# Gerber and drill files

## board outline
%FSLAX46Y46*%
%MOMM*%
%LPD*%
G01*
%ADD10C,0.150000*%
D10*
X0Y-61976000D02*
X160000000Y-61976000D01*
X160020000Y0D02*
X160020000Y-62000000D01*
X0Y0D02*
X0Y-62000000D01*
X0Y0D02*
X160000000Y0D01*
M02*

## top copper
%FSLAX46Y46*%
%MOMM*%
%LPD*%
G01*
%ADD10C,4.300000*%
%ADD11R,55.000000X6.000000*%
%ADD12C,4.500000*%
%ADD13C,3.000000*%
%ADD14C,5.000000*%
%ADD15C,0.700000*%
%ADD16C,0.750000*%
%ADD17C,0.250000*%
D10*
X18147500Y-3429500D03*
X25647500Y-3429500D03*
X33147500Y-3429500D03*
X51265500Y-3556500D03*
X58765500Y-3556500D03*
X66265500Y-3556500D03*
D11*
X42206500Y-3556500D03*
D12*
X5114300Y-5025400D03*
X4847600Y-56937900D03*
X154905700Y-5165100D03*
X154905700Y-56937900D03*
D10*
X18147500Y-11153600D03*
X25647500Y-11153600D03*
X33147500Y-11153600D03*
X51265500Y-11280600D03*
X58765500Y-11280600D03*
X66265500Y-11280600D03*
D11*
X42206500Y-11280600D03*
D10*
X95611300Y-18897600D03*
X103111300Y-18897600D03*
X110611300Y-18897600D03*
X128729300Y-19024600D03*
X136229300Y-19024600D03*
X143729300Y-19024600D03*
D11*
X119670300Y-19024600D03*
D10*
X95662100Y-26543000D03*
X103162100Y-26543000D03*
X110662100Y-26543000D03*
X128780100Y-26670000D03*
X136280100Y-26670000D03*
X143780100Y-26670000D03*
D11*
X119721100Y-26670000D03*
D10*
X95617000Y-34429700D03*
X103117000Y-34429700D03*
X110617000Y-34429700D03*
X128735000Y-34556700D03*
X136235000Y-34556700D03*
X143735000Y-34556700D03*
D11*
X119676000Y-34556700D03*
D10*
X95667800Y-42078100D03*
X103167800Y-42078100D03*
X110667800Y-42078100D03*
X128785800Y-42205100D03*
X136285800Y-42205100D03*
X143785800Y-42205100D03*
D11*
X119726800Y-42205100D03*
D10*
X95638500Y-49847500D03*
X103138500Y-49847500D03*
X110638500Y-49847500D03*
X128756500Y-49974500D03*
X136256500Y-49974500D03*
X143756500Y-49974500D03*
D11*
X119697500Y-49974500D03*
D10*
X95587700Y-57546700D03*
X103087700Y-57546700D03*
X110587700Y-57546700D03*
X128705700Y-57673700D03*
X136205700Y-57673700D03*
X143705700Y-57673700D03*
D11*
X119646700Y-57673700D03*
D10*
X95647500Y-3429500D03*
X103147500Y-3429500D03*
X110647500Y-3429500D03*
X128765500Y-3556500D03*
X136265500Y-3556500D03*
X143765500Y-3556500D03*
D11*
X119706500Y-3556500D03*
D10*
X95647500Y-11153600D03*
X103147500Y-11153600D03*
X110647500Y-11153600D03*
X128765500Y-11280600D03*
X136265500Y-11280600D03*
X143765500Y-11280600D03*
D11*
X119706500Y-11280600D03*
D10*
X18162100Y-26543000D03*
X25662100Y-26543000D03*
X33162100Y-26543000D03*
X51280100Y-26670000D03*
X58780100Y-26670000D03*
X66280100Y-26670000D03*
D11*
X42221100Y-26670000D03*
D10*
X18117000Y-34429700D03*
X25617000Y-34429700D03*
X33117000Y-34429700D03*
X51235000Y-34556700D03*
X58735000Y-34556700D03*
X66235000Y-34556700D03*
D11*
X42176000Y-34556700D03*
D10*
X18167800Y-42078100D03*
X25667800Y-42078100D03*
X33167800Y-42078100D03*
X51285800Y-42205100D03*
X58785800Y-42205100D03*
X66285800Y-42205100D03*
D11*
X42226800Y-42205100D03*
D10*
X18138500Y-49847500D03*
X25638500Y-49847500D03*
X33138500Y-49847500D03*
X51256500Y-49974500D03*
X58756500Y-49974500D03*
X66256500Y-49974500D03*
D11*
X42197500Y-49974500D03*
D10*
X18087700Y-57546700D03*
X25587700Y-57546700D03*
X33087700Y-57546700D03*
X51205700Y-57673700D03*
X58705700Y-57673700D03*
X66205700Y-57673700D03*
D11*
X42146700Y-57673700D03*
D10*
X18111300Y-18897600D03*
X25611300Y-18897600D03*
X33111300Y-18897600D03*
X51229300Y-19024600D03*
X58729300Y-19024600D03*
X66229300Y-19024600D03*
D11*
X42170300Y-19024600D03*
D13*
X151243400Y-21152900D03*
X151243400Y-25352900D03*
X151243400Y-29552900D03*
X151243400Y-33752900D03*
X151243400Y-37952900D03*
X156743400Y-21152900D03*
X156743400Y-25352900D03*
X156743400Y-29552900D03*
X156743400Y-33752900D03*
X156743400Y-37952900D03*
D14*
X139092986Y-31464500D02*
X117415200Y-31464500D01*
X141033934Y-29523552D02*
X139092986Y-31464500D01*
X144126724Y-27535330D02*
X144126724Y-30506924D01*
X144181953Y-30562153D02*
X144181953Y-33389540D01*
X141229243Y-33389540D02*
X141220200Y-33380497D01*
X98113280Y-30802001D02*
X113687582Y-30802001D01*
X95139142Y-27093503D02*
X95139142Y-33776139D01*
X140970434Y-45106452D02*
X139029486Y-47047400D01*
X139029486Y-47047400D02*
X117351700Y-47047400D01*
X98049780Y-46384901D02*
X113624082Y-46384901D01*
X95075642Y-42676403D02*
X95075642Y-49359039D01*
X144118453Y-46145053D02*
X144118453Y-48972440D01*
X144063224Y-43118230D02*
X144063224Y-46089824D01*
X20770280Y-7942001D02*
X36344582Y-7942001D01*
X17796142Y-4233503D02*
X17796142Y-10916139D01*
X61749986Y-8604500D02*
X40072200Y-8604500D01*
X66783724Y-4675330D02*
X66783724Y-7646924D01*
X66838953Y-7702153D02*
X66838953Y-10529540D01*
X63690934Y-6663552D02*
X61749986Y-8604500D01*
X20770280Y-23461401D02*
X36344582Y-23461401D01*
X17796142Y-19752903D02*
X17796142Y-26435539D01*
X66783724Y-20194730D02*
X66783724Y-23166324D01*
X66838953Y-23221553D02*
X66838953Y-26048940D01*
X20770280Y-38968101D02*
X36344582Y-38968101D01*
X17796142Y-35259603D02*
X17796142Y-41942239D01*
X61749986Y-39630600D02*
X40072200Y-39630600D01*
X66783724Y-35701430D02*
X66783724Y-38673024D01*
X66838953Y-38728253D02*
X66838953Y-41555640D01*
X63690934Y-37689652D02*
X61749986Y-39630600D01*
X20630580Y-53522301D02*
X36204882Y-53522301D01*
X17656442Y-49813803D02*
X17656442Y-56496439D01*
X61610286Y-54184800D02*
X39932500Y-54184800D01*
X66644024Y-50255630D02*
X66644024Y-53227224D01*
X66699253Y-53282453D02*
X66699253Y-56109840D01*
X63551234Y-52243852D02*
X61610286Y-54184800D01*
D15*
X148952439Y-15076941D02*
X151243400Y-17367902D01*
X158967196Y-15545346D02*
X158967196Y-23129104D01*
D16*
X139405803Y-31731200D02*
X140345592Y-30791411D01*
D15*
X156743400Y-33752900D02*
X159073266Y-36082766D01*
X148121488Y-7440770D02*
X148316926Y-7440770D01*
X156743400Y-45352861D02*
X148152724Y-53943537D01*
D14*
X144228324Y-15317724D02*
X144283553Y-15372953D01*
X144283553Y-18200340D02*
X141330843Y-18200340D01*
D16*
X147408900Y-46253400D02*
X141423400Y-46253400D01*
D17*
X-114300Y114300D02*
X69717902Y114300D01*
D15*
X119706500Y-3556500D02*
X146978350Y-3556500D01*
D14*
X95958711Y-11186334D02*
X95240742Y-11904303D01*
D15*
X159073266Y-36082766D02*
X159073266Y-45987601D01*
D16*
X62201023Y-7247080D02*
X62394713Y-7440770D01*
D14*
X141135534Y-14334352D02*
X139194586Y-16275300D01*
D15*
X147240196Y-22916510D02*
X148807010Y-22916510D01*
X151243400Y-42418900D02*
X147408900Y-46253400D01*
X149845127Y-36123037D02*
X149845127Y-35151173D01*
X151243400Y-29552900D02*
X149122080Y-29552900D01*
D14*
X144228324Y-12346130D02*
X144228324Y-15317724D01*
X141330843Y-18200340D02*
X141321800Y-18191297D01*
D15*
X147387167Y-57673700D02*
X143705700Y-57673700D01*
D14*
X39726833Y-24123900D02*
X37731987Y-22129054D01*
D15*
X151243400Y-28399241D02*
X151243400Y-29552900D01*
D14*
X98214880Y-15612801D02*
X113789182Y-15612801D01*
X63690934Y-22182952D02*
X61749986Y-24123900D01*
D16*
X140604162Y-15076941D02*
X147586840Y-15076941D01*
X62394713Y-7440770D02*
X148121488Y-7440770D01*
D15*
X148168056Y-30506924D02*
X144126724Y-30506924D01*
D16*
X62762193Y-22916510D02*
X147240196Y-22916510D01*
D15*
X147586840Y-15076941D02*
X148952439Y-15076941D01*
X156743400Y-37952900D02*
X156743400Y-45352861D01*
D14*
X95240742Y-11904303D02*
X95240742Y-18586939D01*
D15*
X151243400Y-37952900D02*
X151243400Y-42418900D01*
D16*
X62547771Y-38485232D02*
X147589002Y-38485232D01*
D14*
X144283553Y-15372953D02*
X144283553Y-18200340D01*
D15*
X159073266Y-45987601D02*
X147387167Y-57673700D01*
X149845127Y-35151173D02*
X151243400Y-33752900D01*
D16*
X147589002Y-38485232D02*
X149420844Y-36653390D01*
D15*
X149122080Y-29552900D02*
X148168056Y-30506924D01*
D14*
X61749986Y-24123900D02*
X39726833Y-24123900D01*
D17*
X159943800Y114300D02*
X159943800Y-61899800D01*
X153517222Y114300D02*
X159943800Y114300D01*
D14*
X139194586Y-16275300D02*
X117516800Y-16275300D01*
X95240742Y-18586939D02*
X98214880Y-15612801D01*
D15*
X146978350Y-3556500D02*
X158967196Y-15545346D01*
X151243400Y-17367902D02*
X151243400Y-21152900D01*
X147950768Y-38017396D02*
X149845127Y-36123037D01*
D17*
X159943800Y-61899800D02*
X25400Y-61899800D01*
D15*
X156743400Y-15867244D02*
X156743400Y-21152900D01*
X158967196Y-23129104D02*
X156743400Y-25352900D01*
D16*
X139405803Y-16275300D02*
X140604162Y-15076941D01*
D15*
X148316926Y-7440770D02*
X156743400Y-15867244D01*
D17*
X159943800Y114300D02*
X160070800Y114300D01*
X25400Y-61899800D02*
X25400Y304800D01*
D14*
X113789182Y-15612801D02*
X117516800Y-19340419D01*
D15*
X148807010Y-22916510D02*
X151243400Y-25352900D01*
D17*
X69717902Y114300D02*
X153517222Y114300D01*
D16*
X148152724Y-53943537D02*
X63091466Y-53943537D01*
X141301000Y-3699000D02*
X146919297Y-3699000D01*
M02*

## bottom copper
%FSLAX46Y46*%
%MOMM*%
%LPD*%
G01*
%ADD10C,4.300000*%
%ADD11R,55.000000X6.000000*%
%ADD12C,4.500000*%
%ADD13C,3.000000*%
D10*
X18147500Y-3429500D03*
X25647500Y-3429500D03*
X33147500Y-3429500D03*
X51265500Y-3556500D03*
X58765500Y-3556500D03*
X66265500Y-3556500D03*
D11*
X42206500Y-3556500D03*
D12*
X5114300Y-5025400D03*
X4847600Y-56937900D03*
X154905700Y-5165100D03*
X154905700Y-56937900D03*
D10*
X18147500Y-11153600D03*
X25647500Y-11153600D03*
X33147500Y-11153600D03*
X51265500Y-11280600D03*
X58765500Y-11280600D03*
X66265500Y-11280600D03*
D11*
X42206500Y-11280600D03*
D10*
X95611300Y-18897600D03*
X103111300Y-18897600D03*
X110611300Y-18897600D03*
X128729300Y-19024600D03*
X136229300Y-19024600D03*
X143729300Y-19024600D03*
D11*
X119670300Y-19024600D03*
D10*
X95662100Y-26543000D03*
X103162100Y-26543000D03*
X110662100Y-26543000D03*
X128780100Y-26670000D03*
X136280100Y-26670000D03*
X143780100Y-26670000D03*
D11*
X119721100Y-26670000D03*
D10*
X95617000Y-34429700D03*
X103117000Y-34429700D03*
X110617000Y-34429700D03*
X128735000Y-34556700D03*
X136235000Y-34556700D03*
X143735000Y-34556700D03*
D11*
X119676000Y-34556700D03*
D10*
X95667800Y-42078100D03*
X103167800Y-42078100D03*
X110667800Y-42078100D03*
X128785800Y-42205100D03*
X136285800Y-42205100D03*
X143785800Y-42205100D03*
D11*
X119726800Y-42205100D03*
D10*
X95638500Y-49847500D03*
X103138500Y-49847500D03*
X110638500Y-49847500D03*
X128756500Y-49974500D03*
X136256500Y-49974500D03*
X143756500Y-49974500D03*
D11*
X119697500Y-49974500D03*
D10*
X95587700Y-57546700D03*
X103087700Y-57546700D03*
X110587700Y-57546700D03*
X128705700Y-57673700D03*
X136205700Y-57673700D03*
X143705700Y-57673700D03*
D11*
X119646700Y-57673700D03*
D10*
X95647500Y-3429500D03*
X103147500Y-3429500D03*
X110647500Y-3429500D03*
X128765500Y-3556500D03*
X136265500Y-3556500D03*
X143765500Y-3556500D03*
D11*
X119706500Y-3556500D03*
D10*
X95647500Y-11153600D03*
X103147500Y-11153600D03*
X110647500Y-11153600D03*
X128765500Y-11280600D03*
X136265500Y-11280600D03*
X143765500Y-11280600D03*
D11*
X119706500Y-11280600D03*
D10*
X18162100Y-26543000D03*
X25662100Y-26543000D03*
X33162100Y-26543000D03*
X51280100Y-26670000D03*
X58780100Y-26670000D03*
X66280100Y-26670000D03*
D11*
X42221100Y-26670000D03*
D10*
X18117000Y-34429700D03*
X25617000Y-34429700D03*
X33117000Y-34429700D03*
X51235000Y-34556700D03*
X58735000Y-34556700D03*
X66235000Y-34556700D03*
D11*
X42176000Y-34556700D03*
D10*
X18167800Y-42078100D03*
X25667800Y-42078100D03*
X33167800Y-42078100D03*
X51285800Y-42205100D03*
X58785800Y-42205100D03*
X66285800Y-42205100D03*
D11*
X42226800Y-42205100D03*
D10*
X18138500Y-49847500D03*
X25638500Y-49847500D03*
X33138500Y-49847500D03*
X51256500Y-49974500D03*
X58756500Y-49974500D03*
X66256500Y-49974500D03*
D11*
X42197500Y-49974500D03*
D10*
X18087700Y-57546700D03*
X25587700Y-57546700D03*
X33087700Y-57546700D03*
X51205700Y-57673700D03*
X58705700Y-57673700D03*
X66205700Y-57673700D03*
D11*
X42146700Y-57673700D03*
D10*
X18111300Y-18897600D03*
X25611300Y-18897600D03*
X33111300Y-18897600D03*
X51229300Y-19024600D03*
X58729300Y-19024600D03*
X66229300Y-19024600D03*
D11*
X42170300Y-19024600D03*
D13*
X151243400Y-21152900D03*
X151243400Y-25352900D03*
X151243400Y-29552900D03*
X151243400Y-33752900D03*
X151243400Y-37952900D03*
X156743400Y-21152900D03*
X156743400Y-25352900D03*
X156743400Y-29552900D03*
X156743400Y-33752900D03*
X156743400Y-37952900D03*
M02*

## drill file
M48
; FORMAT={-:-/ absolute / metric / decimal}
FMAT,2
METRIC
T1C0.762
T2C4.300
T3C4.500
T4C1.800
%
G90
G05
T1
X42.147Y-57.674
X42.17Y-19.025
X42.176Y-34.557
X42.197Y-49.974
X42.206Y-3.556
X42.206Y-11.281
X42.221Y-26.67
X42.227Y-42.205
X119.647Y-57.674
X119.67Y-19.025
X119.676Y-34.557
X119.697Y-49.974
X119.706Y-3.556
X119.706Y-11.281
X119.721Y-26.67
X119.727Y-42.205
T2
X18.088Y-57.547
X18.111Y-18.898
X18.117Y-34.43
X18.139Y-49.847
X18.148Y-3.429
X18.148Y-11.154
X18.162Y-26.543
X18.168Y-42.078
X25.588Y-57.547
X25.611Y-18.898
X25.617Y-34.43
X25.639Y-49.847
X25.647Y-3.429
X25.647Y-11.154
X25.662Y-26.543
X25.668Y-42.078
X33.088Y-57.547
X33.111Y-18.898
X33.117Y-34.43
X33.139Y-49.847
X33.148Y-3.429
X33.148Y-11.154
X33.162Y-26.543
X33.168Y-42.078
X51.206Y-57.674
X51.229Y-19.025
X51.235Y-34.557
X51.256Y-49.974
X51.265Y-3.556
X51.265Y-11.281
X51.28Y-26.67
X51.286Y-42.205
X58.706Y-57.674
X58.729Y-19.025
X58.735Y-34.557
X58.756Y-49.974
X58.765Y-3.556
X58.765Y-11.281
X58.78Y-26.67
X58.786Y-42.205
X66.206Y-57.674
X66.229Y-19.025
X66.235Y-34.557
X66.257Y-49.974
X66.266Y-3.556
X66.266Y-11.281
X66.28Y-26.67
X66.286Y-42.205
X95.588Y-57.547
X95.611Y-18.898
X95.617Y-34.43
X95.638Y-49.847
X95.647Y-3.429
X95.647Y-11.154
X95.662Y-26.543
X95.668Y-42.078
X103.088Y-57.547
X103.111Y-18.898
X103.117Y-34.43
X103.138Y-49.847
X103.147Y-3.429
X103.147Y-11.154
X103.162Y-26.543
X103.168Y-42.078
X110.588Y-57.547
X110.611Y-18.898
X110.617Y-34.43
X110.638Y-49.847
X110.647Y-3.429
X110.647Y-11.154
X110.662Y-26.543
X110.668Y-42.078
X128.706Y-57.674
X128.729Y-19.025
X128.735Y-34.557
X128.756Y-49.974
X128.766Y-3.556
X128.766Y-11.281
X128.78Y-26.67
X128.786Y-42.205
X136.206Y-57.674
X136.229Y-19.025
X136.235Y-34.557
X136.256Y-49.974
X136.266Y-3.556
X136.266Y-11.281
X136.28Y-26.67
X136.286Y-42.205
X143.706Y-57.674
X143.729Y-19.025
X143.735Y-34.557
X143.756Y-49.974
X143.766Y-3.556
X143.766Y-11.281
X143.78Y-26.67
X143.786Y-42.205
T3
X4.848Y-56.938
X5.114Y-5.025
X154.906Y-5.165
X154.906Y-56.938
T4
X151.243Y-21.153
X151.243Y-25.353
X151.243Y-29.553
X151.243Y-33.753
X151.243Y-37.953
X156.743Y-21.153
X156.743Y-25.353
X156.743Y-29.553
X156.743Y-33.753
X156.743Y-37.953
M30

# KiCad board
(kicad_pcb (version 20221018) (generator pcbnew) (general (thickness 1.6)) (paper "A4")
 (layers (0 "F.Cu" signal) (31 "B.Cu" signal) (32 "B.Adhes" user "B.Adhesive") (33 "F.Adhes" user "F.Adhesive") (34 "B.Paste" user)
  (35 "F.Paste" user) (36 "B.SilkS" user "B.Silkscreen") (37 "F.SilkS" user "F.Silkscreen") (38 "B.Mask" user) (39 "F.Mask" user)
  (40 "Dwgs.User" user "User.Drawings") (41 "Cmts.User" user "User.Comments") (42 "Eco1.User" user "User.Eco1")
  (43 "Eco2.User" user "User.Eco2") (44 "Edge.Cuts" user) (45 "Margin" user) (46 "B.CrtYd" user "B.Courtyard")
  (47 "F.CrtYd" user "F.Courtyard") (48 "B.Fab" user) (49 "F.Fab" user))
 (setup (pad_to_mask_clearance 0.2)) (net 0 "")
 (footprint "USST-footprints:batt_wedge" (layer "F.Cu") (at 42.2065 3.5565)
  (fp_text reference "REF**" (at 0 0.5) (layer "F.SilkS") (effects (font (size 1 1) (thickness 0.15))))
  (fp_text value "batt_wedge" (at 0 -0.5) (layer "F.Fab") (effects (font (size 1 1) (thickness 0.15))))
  (pad "" thru_hole circle (at -24.059 -0.127) (size 4.3 4.3) (drill 4.3) (layers "*.Cu" "*.Mask"))
  (pad "" thru_hole circle (at -16.559 -0.127) (size 4.3 4.3) (drill 4.3) (layers "*.Cu" "*.Mask"))
  (pad "" thru_hole circle (at -9.059 -0.127) (size 4.3 4.3) (drill 4.3) (layers "*.Cu" "*.Mask"))
  (pad "" thru_hole circle (at 9.059 0) (size 4.3 4.3) (drill 4.3) (layers "*.Cu" "*.Mask"))
  (pad "" thru_hole circle (at 16.559 0) (size 4.3 4.3) (drill 4.3) (layers "*.Cu" "*.Mask"))
  (pad "" thru_hole circle (at 24.059 0) (size 4.3 4.3) (drill 4.3) (layers "*.Cu" "*.Mask"))
  (pad "1" thru_hole rect (at 0 0) (size 55 6) (drill 0.762) (layers "F.Cu" "F.Paste")))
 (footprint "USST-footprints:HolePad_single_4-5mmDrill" (layer "F.Cu") (at 5.1143 5.0254)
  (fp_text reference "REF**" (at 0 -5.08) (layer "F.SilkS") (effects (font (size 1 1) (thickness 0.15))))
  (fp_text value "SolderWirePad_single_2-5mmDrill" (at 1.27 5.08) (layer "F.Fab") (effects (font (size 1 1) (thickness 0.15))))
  (pad "" thru_hole circle (at 0 0) (size 4.5 4.5) (drill 4.5) (layers "*.Cu" "*.Mask")))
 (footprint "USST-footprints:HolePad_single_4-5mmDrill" (layer "F.Cu") (at 4.8476 56.9379)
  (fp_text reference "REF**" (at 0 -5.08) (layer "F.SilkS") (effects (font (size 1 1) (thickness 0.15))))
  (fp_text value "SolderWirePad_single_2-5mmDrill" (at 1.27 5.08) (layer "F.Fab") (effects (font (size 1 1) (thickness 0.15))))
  (pad "" thru_hole circle (at 0 0) (size 4.5 4.5) (drill 4.5) (layers "*.Cu" "*.Mask")))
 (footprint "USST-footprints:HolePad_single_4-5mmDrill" (layer "F.Cu") (at 154.9057 5.1651)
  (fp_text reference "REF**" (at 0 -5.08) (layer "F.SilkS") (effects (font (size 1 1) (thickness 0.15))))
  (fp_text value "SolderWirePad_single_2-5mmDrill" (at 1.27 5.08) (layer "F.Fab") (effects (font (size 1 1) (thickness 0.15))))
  (pad "" thru_hole circle (at 0 0) (size 4.5 4.5) (drill 4.5) (layers "*.Cu" "*.Mask")))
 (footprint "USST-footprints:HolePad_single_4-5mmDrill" (layer "F.Cu") (at 154.9057 56.9379)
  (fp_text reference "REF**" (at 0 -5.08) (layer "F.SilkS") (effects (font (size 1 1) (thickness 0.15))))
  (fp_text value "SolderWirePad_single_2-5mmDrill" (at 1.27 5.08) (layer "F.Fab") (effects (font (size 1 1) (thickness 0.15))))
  (pad "" thru_hole circle (at 0 0) (size 4.5 4.5) (drill 4.5) (layers "*.Cu" "*.Mask")))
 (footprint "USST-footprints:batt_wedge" (layer "F.Cu") (at 42.2065 11.2806)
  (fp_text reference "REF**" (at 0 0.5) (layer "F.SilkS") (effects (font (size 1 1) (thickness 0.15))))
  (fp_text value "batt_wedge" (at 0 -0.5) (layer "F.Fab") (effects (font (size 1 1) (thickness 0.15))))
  (pad "" thru_hole circle (at -24.059 -0.127) (size 4.3 4.3) (drill 4.3) (layers "*.Cu" "*.Mask"))
  (pad "" thru_hole circle (at -16.559 -0.127) (size 4.3 4.3) (drill 4.3) (layers "*.Cu" "*.Mask"))
  (pad "" thru_hole circle (at -9.059 -0.127) (size 4.3 4.3) (drill 4.3) (layers "*.Cu" "*.Mask"))
  (pad "" thru_hole circle (at 9.059 0) (size 4.3 4.3) (drill 4.3) (layers "*.Cu" "*.Mask"))
  (pad "" thru_hole circle (at 16.559 0) (size 4.3 4.3) (drill 4.3) (layers "*.Cu" "*.Mask"))
  (pad "" thru_hole circle (at 24.059 0) (size 4.3 4.3) (drill 4.3) (layers "*.Cu" "*.Mask"))
  (pad "1" thru_hole rect (at 0 0) (size 55 6) (drill 0.762) (layers "F.Cu" "F.Paste")))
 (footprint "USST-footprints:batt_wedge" (layer "F.Cu") (at 119.6703 19.0246)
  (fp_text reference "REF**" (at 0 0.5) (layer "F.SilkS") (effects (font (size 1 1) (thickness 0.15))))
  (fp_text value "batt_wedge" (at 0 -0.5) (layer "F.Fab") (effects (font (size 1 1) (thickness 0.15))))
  (pad "" thru_hole circle (at -24.059 -0.127) (size 4.3 4.3) (drill 4.3) (layers "*.Cu" "*.Mask"))
  (pad "" thru_hole circle (at -16.559 -0.127) (size 4.3 4.3) (drill 4.3) (layers "*.Cu" "*.Mask"))
  (pad "" thru_hole circle (at -9.059 -0.127) (size 4.3 4.3) (drill 4.3) (layers "*.Cu" "*.Mask"))
  (pad "" thru_hole circle (at 9.059 0) (size 4.3 4.3) (drill 4.3) (layers "*.Cu" "*.Mask"))
  (pad "" thru_hole circle (at 16.559 0) (size 4.3 4.3) (drill 4.3) (layers "*.Cu" "*.Mask"))
  (pad "" thru_hole circle (at 24.059 0) (size 4.3 4.3) (drill 4.3) (layers "*.Cu" "*.Mask"))
  (pad "1" thru_hole rect (at 0 0) (size 55 6) (drill 0.762) (layers "F.Cu" "F.Paste")))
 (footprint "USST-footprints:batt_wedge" (layer "F.Cu") (at 119.7211 26.67)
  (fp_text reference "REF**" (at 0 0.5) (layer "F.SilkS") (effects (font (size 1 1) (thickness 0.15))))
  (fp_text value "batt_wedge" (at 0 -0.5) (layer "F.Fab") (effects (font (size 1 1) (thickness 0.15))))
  (pad "" thru_hole circle (at -24.059 -0.127) (size 4.3 4.3) (drill 4.3) (layers "*.Cu" "*.Mask"))
  (pad "" thru_hole circle (at -16.559 -0.127) (size 4.3 4.3) (drill 4.3) (layers "*.Cu" "*.Mask"))
  (pad "" thru_hole circle (at -9.059 -0.127) (size 4.3 4.3) (drill 4.3) (layers "*.Cu" "*.Mask"))
  (pad "" thru_hole circle (at 9.059 0) (size 4.3 4.3) (drill 4.3) (layers "*.Cu" "*.Mask"))
  (pad "" thru_hole circle (at 16.559 0) (size 4.3 4.3) (drill 4.3) (layers "*.Cu" "*.Mask"))
  (pad "" thru_hole circle (at 24.059 0) (size 4.3 4.3) (drill 4.3) (layers "*.Cu" "*.Mask"))
  (pad "1" thru_hole rect (at 0 0) (size 55 6) (drill 0.762) (layers "F.Cu" "F.Paste")))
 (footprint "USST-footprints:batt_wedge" (layer "F.Cu") (at 119.676 34.5567)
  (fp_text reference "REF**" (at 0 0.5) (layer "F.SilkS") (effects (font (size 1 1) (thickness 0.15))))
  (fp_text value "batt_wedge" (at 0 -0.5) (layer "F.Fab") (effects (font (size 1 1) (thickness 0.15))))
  (pad "" thru_hole circle (at -24.059 -0.127) (size 4.3 4.3) (drill 4.3) (layers "*.Cu" "*.Mask"))
  (pad "" thru_hole circle (at -16.559 -0.127) (size 4.3 4.3) (drill 4.3) (layers "*.Cu" "*.Mask"))
  (pad "" thru_hole circle (at -9.059 -0.127) (size 4.3 4.3) (drill 4.3) (layers "*.Cu" "*.Mask"))
  (pad "" thru_hole circle (at 9.059 0) (size 4.3 4.3) (drill 4.3) (layers "*.Cu" "*.Mask"))
  (pad "" thru_hole circle (at 16.559 0) (size 4.3 4.3) (drill 4.3) (layers "*.Cu" "*.Mask"))
  (pad "" thru_hole circle (at 24.059 0) (size 4.3 4.3) (drill 4.3) (layers "*.Cu" "*.Mask"))
  (pad "1" thru_hole rect (at 0 0) (size 55 6) (drill 0.762) (layers "F.Cu" "F.Paste")))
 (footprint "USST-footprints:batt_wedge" (layer "F.Cu") (at 119.7268 42.2051)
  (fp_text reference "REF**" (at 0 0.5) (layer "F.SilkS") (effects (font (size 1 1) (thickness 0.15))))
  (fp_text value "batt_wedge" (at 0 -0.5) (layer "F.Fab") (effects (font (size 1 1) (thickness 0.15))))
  (pad "" thru_hole circle (at -24.059 -0.127) (size 4.3 4.3) (drill 4.3) (layers "*.Cu" "*.Mask"))
  (pad "" thru_hole circle (at -16.559 -0.127) (size 4.3 4.3) (drill 4.3) (layers "*.Cu" "*.Mask"))
  (pad "" thru_hole circle (at -9.059 -0.127) (size 4.3 4.3) (drill 4.3) (layers "*.Cu" "*.Mask"))
  (pad "" thru_hole circle (at 9.059 0) (size 4.3 4.3) (drill 4.3) (layers "*.Cu" "*.Mask"))
  (pad "" thru_hole circle (at 16.559 0) (size 4.3 4.3) (drill 4.3) (layers "*.Cu" "*.Mask"))
  (pad "" thru_hole circle (at 24.059 0) (size 4.3 4.3) (drill 4.3) (layers "*.Cu" "*.Mask"))
  (pad "1" thru_hole rect (at 0 0) (size 55 6) (drill 0.762) (layers "F.Cu" "F.Paste")))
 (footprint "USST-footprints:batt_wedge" (layer "F.Cu") (at 119.6975 49.9745)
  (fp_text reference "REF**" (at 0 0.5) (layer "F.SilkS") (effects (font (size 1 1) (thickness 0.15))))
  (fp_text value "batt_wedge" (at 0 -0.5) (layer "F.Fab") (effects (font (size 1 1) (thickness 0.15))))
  (pad "" thru_hole circle (at -24.059 -0.127) (size 4.3 4.3) (drill 4.3) (layers "*.Cu" "*.Mask"))
  (pad "" thru_hole circle (at -16.559 -0.127) (size 4.3 4.3) (drill 4.3) (layers "*.Cu" "*.Mask"))
  (pad "" thru_hole circle (at -9.059 -0.127) (size 4.3 4.3) (drill 4.3) (layers "*.Cu" "*.Mask"))
  (pad "" thru_hole circle (at 9.059 0) (size 4.3 4.3) (drill 4.3) (layers "*.Cu" "*.Mask"))
  (pad "" thru_hole circle (at 16.559 0) (size 4.3 4.3) (drill 4.3) (layers "*.Cu" "*.Mask"))
  (pad "" thru_hole circle (at 24.059 0) (size 4.3 4.3) (drill 4.3) (layers "*.Cu" "*.Mask"))
  (pad "1" thru_hole rect (at 0 0) (size 55 6) (drill 0.762) (layers "F.Cu" "F.Paste")))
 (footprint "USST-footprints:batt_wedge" (layer "F.Cu") (at 119.6467 57.6737)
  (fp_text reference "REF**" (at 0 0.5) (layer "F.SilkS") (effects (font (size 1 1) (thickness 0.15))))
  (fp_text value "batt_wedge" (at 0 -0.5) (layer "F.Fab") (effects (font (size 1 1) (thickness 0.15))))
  (pad "" thru_hole circle (at -24.059 -0.127) (size 4.3 4.3) (drill 4.3) (layers "*.Cu" "*.Mask"))
  (pad "" thru_hole circle (at -16.559 -0.127) (size 4.3 4.3) (drill 4.3) (layers "*.Cu" "*.Mask"))
  (pad "" thru_hole circle (at -9.059 -0.127) (size 4.3 4.3) (drill 4.3) (layers "*.Cu" "*.Mask"))
  (pad "" thru_hole circle (at 9.059 0) (size 4.3 4.3) (drill 4.3) (layers "*.Cu" "*.Mask"))
  (pad "" thru_hole circle (at 16.559 0) (size 4.3 4.3) (drill 4.3) (layers "*.Cu" "*.Mask"))
  (pad "" thru_hole circle (at 24.059 0) (size 4.3 4.3) (drill 4.3) (layers "*.Cu" "*.Mask"))
  (pad "1" thru_hole rect (at 0 0) (size 55 6) (drill 0.762) (layers "F.Cu" "F.Paste")))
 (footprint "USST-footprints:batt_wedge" (layer "F.Cu") (at 119.7065 3.5565)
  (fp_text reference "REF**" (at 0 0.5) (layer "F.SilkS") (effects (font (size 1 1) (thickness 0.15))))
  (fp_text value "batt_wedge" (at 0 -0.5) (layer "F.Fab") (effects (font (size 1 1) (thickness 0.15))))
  (pad "" thru_hole circle (at -24.059 -0.127) (size 4.3 4.3) (drill 4.3) (layers "*.Cu" "*.Mask"))
  (pad "" thru_hole circle (at -16.559 -0.127) (size 4.3 4.3) (drill 4.3) (layers "*.Cu" "*.Mask"))
  (pad "" thru_hole circle (at -9.059 -0.127) (size 4.3 4.3) (drill 4.3) (layers "*.Cu" "*.Mask"))
  (pad "" thru_hole circle (at 9.059 0) (size 4.3 4.3) (drill 4.3) (layers "*.Cu" "*.Mask"))
  (pad "" thru_hole circle (at 16.559 0) (size 4.3 4.3) (drill 4.3) (layers "*.Cu" "*.Mask"))
  (pad "" thru_hole circle (at 24.059 0) (size 4.3 4.3) (drill 4.3) (layers "*.Cu" "*.Mask"))
  (pad "1" thru_hole rect (at 0 0) (size 55 6) (drill 0.762) (layers "F.Cu" "F.Paste")))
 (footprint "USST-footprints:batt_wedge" (layer "F.Cu") (at 119.7065 11.2806)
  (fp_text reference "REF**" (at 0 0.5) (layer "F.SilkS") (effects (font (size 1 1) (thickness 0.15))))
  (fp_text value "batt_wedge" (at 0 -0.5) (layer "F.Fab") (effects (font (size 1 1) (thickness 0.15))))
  (pad "" thru_hole circle (at -24.059 -0.127) (size 4.3 4.3) (drill 4.3) (layers "*.Cu" "*.Mask"))
  (pad "" thru_hole circle (at -16.559 -0.127) (size 4.3 4.3) (drill 4.3) (layers "*.Cu" "*.Mask"))
  (pad "" thru_hole circle (at -9.059 -0.127) (size 4.3 4.3) (drill 4.3) (layers "*.Cu" "*.Mask"))
  (pad "" thru_hole circle (at 9.059 0) (size 4.3 4.3) (drill 4.3) (layers "*.Cu" "*.Mask"))
  (pad "" thru_hole circle (at 16.559 0) (size 4.3 4.3) (drill 4.3) (layers "*.Cu" "*.Mask"))
  (pad "" thru_hole circle (at 24.059 0) (size 4.3 4.3) (drill 4.3) (layers "*.Cu" "*.Mask"))
  (pad "1" thru_hole rect (at 0 0) (size 55 6) (drill 0.762) (layers "F.Cu" "F.Paste")))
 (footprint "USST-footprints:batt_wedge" (layer "F.Cu") (at 42.2211 26.67)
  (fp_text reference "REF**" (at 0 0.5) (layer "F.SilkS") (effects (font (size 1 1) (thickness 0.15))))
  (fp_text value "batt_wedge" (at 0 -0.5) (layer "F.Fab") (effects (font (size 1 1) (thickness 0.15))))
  (pad "" thru_hole circle (at -24.059 -0.127) (size 4.3 4.3) (drill 4.3) (layers "*.Cu" "*.Mask"))
  (pad "" thru_hole circle (at -16.559 -0.127) (size 4.3 4.3) (drill 4.3) (layers "*.Cu" "*.Mask"))
  (pad "" thru_hole circle (at -9.059 -0.127) (size 4.3 4.3) (drill 4.3) (layers "*.Cu" "*.Mask"))
  (pad "" thru_hole circle (at 9.059 0) (size 4.3 4.3) (drill 4.3) (layers "*.Cu" "*.Mask"))
  (pad "" thru_hole circle (at 16.559 0) (size 4.3 4.3) (drill 4.3) (layers "*.Cu" "*.Mask"))
  (pad "" thru_hole circle (at 24.059 0) (size 4.3 4.3) (drill 4.3) (layers "*.Cu" "*.Mask"))
  (pad "1" thru_hole rect (at 0 0) (size 55 6) (drill 0.762) (layers "F.Cu" "F.Paste")))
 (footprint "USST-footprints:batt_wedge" (layer "F.Cu") (at 42.176 34.5567)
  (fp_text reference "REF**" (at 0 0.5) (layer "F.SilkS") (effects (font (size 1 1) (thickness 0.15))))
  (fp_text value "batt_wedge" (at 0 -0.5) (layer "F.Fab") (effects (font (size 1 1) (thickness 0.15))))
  (pad "" thru_hole circle (at -24.059 -0.127) (size 4.3 4.3) (drill 4.3) (layers "*.Cu" "*.Mask"))
  (pad "" thru_hole circle (at -16.559 -0.127) (size 4.3 4.3) (drill 4.3) (layers "*.Cu" "*.Mask"))
  (pad "" thru_hole circle (at -9.059 -0.127) (size 4.3 4.3) (drill 4.3) (layers "*.Cu" "*.Mask"))
  (pad "" thru_hole circle (at 9.059 0) (size 4.3 4.3) (drill 4.3) (layers "*.Cu" "*.Mask"))
  (pad "" thru_hole circle (at 16.559 0) (size 4.3 4.3) (drill 4.3) (layers "*.Cu" "*.Mask"))
  (pad "" thru_hole circle (at 24.059 0) (size 4.3 4.3) (drill 4.3) (layers "*.Cu" "*.Mask"))
  (pad "1" thru_hole rect (at 0 0) (size 55 6) (drill 0.762) (layers "F.Cu" "F.Paste")))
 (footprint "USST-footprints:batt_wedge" (layer "F.Cu") (at 42.2268 42.2051)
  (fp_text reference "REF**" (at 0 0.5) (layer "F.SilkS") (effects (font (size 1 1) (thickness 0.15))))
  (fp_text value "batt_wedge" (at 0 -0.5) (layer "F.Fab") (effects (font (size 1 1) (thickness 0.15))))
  (pad "" thru_hole circle (at -24.059 -0.127) (size 4.3 4.3) (drill 4.3) (layers "*.Cu" "*.Mask"))
  (pad "" thru_hole circle (at -16.559 -0.127) (size 4.3 4.3) (drill 4.3) (layers "*.Cu" "*.Mask"))
  (pad "" thru_hole circle (at -9.059 -0.127) (size 4.3 4.3) (drill 4.3) (layers "*.Cu" "*.Mask"))
  (pad "" thru_hole circle (at 9.059 0) (size 4.3 4.3) (drill 4.3) (layers "*.Cu" "*.Mask"))
  (pad "" thru_hole circle (at 16.559 0) (size 4.3 4.3) (drill 4.3) (layers "*.Cu" "*.Mask"))
  (pad "" thru_hole circle (at 24.059 0) (size 4.3 4.3) (drill 4.3) (layers "*.Cu" "*.Mask"))
  (pad "1" thru_hole rect (at 0 0) (size 55 6) (drill 0.762) (layers "F.Cu" "F.Paste")))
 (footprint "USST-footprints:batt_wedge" (layer "F.Cu") (at 42.1975 49.9745)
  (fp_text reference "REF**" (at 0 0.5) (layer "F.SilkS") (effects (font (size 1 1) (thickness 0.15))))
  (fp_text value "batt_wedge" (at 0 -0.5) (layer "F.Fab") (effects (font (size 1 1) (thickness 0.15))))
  (pad "" thru_hole circle (at -24.059 -0.127) (size 4.3 4.3) (drill 4.3) (layers "*.Cu" "*.Mask"))
  (pad "" thru_hole circle (at -16.559 -0.127) (size 4.3 4.3) (drill 4.3) (layers "*.Cu" "*.Mask"))
  (pad "" thru_hole circle (at -9.059 -0.127) (size 4.3 4.3) (drill 4.3) (layers "*.Cu" "*.Mask"))
  (pad "" thru_hole circle (at 9.059 0) (size 4.3 4.3) (drill 4.3) (layers "*.Cu" "*.Mask"))
  (pad "" thru_hole circle (at 16.559 0) (size 4.3 4.3) (drill 4.3) (layers "*.Cu" "*.Mask"))
  (pad "" thru_hole circle (at 24.059 0) (size 4.3 4.3) (drill 4.3) (layers "*.Cu" "*.Mask"))
  (pad "1" thru_hole rect (at 0 0) (size 55 6) (drill 0.762) (layers "F.Cu" "F.Paste")))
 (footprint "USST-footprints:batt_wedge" (layer "F.Cu") (at 42.1467 57.6737)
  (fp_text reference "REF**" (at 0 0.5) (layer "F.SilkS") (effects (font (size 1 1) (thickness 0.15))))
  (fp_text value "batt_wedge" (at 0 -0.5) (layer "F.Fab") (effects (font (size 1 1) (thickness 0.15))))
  (pad "" thru_hole circle (at -24.059 -0.127) (size 4.3 4.3) (drill 4.3) (layers "*.Cu" "*.Mask"))
  (pad "" thru_hole circle (at -16.559 -0.127) (size 4.3 4.3) (drill 4.3) (layers "*.Cu" "*.Mask"))
  (pad "" thru_hole circle (at -9.059 -0.127) (size 4.3 4.3) (drill 4.3) (layers "*.Cu" "*.Mask"))
  (pad "" thru_hole circle (at 9.059 0) (size 4.3 4.3) (drill 4.3) (layers "*.Cu" "*.Mask"))
  (pad "" thru_hole circle (at 16.559 0) (size 4.3 4.3) (drill 4.3) (layers "*.Cu" "*.Mask"))
  (pad "" thru_hole circle (at 24.059 0) (size 4.3 4.3) (drill 4.3) (layers "*.Cu" "*.Mask"))
  (pad "1" thru_hole rect (at 0 0) (size 55 6) (drill 0.762) (layers "F.Cu" "F.Paste")))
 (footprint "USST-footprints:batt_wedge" (layer "F.Cu") (at 42.1703 19.0246)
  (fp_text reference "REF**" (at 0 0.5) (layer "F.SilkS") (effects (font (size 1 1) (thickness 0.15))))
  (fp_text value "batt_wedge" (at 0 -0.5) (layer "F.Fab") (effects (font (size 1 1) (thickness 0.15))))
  (pad "" thru_hole circle (at -24.059 -0.127) (size 4.3 4.3) (drill 4.3) (layers "*.Cu" "*.Mask"))
  (pad "" thru_hole circle (at -16.559 -0.127) (size 4.3 4.3) (drill 4.3) (layers "*.Cu" "*.Mask"))
  (pad "" thru_hole circle (at -9.059 -0.127) (size 4.3 4.3) (drill 4.3) (layers "*.Cu" "*.Mask"))
  (pad "" thru_hole circle (at 9.059 0) (size 4.3 4.3) (drill 4.3) (layers "*.Cu" "*.Mask"))
  (pad "" thru_hole circle (at 16.559 0) (size 4.3 4.3) (drill 4.3) (layers "*.Cu" "*.Mask"))
  (pad "" thru_hole circle (at 24.059 0) (size 4.3 4.3) (drill 4.3) (layers "*.Cu" "*.Mask"))
  (pad "1" thru_hole rect (at 0 0) (size 55 6) (drill 0.762) (layers "F.Cu" "F.Paste")))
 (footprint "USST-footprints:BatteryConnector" (layer "F.Cu") (at 151.2434 37.9529)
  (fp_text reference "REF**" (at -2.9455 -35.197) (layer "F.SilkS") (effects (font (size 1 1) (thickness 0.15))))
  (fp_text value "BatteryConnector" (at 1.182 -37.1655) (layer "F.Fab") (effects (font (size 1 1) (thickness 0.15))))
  (pad "" np_thru_hole circle (at 0 -16.8) (size 3 3) (drill 1.8) (layers "*.Cu"))
  (pad "" np_thru_hole circle (at 0 -12.6) (size 3 3) (drill 1.8) (layers "*.Cu"))
  (pad "" np_thru_hole circle (at 0 -8.4) (size 3 3) (drill 1.8) (layers "*.Cu"))
  (pad "" np_thru_hole circle (at 0 -4.2) (size 3 3) (drill 1.8) (layers "*.Cu"))
  (pad "" np_thru_hole circle (at 0 0) (size 3 3) (drill 1.8) (layers "*.Cu"))
  (pad "" np_thru_hole circle (at 5.5 -16.8) (size 3 3) (drill 1.8) (layers "*.Cu"))
  (pad "" np_thru_hole circle (at 5.5 -12.6) (size 3 3) (drill 1.8) (layers "*.Cu"))
  (pad "" np_thru_hole circle (at 5.5 -8.4) (size 3 3) (drill 1.8) (layers "*.Cu"))
  (pad "" np_thru_hole circle (at 5.5 -4.2) (size 3 3) (drill 1.8) (layers "*.Cu"))
  (pad "" np_thru_hole circle (at 5.5 0) (size 3 3) (drill 1.8) (layers "*.Cu")))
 (gr_line (start 0 61.976) (end 160 61.976) (stroke (width 0.15) (type solid)) (layer "Edge.Cuts"))
 (gr_line (start 160.02 0) (end 160.02 62) (stroke (width 0.15) (type solid)) (layer "Edge.Cuts"))
 (gr_line (start 0 0) (end 0 62) (stroke (width 0.15) (type solid)) (layer "Edge.Cuts"))
 (gr_line (start 0 0) (end 160 0) (stroke (width 0.15) (type solid)) (layer "Edge.Cuts"))
 (segment (start 139.092986 31.4645) (end 117.4152 31.4645) (width 5) (layer "F.Cu") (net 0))
 (segment (start 141.033934 29.523552) (end 139.092986 31.4645) (width 5) (layer "F.Cu") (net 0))
 (segment (start 144.126724 27.53533) (end 144.126724 30.506924) (width 5) (layer "F.Cu") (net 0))
 (segment (start 144.181953 30.562153) (end 144.181953 33.38954) (width 5) (layer "F.Cu") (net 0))
 (segment (start 141.229243 33.38954) (end 141.2202 33.380497) (width 5) (layer "F.Cu") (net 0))
 (segment (start 98.11328 30.802001) (end 113.687582 30.802001) (width 5) (layer "F.Cu") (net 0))
 (segment (start 95.139142 27.093503) (end 95.139142 33.776139) (width 5) (layer "F.Cu") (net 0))
 (segment (start 140.970434 45.106452) (end 139.029486 47.0474) (width 5) (layer "F.Cu") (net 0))
 (segment (start 139.029486 47.0474) (end 117.3517 47.0474) (width 5) (layer "F.Cu") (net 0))
 (segment (start 98.04978 46.384901) (end 113.624082 46.384901) (width 5) (layer "F.Cu") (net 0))
 (segment (start 95.075642 42.676403) (end 95.075642 49.359039) (width 5) (layer "F.Cu") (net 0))
 (segment (start 144.118453 46.145053) (end 144.118453 48.97244) (width 5) (layer "F.Cu") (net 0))
 (segment (start 144.063224 43.11823) (end 144.063224 46.089824) (width 5) (layer "F.Cu") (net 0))
 (segment (start 20.77028 7.942001) (end 36.344582 7.942001) (width 5) (layer "F.Cu") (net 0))
 (segment (start 17.796142 4.233503) (end 17.796142 10.916139) (width 5) (layer "F.Cu") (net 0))
 (segment (start 61.749986 8.6045) (end 40.0722 8.6045) (width 5) (layer "F.Cu") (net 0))
 (segment (start 66.783724 4.67533) (end 66.783724 7.646924) (width 5) (layer "F.Cu") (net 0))
 (segment (start 66.838953 7.702153) (end 66.838953 10.52954) (width 5) (layer "F.Cu") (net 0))
 (segment (start 63.690934 6.663552) (end 61.749986 8.6045) (width 5) (layer "F.Cu") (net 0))
 (segment (start 20.77028 23.461401) (end 36.344582 23.461401) (width 5) (layer "F.Cu") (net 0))
 (segment (start 17.796142 19.752903) (end 17.796142 26.435539) (width 5) (layer "F.Cu") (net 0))
 (segment (start 66.783724 20.19473) (end 66.783724 23.166324) (width 5) (layer "F.Cu") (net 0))
 (segment (start 66.838953 23.221553) (end 66.838953 26.04894) (width 5) (layer "F.Cu") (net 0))
 (segment (start 20.77028 38.968101) (end 36.344582 38.968101) (width 5) (layer "F.Cu") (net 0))
 (segment (start 17.796142 35.259603) (end 17.796142 41.942239) (width 5) (layer "F.Cu") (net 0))
 (segment (start 61.749986 39.6306) (end 40.0722 39.6306) (width 5) (layer "F.Cu") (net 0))
 (segment (start 66.783724 35.70143) (end 66.783724 38.673024) (width 5) (layer "F.Cu") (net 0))
 (segment (start 66.838953 38.728253) (end 66.838953 41.55564) (width 5) (layer "F.Cu") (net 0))
 (segment (start 63.690934 37.689652) (end 61.749986 39.6306) (width 5) (layer "F.Cu") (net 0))
 (segment (start 20.63058 53.522301) (end 36.204882 53.522301) (width 5) (layer "F.Cu") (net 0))
 (segment (start 17.656442 49.813803) (end 17.656442 56.496439) (width 5) (layer "F.Cu") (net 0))
 (segment (start 61.610286 54.1848) (end 39.9325 54.1848) (width 5) (layer "F.Cu") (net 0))
 (segment (start 66.644024 50.25563) (end 66.644024 53.227224) (width 5) (layer "F.Cu") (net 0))
 (segment (start 66.699253 53.282453) (end 66.699253 56.10984) (width 5) (layer "F.Cu") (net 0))
 (segment (start 63.551234 52.243852) (end 61.610286 54.1848) (width 5) (layer "F.Cu") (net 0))
 (segment (start 148.952439 15.076941) (end 151.2434 17.367902) (width 0.7) (layer "F.Cu") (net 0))
 (segment (start 158.967196 15.545346) (end 158.967196 23.129104) (width 0.7) (layer "F.Cu") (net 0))
 (segment (start 139.405803 31.7312) (end 140.345592 30.791411) (width 0.75) (layer "F.Cu") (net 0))
 (segment (start 156.7434 33.7529) (end 159.073266 36.082766) (width 0.7) (layer "F.Cu") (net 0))
 (segment (start 148.121488 7.44077) (end 148.316926 7.44077) (width 0.7) (layer "F.Cu") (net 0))
 (segment (start 156.7434 45.352861) (end 148.152724 53.943537) (width 0.7) (layer "F.Cu") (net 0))
 (segment (start 144.228324 15.317724) (end 144.283553 15.372953) (width 5) (layer "F.Cu") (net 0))
 (segment (start 144.283553 18.20034) (end 141.330843 18.20034) (width 5) (layer "F.Cu") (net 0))
 (segment (start 147.4089 46.2534) (end 141.4234 46.2534) (width 0.75) (layer "F.Cu") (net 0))
 (segment (start -0.1143 -0.1143) (end 69.717902 -0.1143) (width 0.25) (layer "F.Cu") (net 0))
 (segment (start 119.7065 3.5565) (end 146.97835 3.5565) (width 0.7) (layer "F.Cu") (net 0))
 (segment (start 95.958711 11.186334) (end 95.240742 11.904303) (width 5) (layer "F.Cu") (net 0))
 (segment (start 159.073266 36.082766) (end 159.073266 45.987601) (width 0.7) (layer "F.Cu") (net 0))
 (segment (start 62.201023 7.24708) (end 62.394713 7.44077) (width 0.75) (layer "F.Cu") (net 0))
 (segment (start 141.135534 14.334352) (end 139.194586 16.2753) (width 5) (layer "F.Cu") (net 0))
 (segment (start 147.240196 22.91651) (end 148.80701 22.91651) (width 0.7) (layer "F.Cu") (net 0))
 (segment (start 151.2434 42.4189) (end 147.4089 46.2534) (width 0.7) (layer "F.Cu") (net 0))
 (segment (start 149.845127 36.123037) (end 149.845127 35.151173) (width 0.7) (layer "F.Cu") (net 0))
 (segment (start 151.2434 29.5529) (end 149.12208 29.5529) (width 0.7) (layer "F.Cu") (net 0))
 (segment (start 144.228324 12.34613) (end 144.228324 15.317724) (width 5) (layer "F.Cu") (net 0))
 (segment (start 141.330843 18.20034) (end 141.3218 18.191297) (width 5) (layer "F.Cu") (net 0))
 (segment (start 147.387167 57.6737) (end 143.7057 57.6737) (width 0.7) (layer "F.Cu") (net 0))
 (segment (start 39.726833 24.1239) (end 37.731987 22.129054) (width 5) (layer "F.Cu") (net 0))
 (segment (start 151.2434 28.399241) (end 151.2434 29.5529) (width 0.7) (layer "F.Cu") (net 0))
 (segment (start 98.21488 15.612801) (end 113.789182 15.612801) (width 5) (layer "F.Cu") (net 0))
 (segment (start 63.690934 22.182952) (end 61.749986 24.1239) (width 5) (layer "F.Cu") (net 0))
 (segment (start 140.604162 15.076941) (end 147.58684 15.076941) (width 0.75) (layer "F.Cu") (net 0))
 (segment (start 62.394713 7.44077) (end 148.121488 7.44077) (width 0.75) (layer "F.Cu") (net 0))
 (segment (start 148.168056 30.506924) (end 144.126724 30.506924) (width 0.7) (layer "F.Cu") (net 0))
 (segment (start 62.762193 22.91651) (end 147.240196 22.91651) (width 0.75) (layer "F.Cu") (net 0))
 (segment (start 147.58684 15.076941) (end 148.952439 15.076941) (width 0.7) (layer "F.Cu") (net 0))
 (segment (start 156.7434 37.9529) (end 156.7434 45.352861) (width 0.7) (layer "F.Cu") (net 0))
 (segment (start 95.240742 11.904303) (end 95.240742 18.586939) (width 5) (layer "F.Cu") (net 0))
 (segment (start 151.2434 37.9529) (end 151.2434 42.4189) (width 0.7) (layer "F.Cu") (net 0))
 (segment (start 62.547771 38.485232) (end 147.589002 38.485232) (width 0.75) (layer "F.Cu") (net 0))
 (segment (start 144.283553 15.372953) (end 144.283553 18.20034) (width 5) (layer "F.Cu") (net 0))
 (segment (start 159.073266 45.987601) (end 147.387167 57.6737) (width 0.7) (layer "F.Cu") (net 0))
 (segment (start 149.845127 35.151173) (end 151.2434 33.7529) (width 0.7) (layer "F.Cu") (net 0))
 (segment (start 147.589002 38.485232) (end 149.420844 36.65339) (width 0.75) (layer "F.Cu") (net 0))
 (segment (start 149.12208 29.5529) (end 148.168056 30.506924) (width 0.7) (layer "F.Cu") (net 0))
 (segment (start 61.749986 24.1239) (end 39.726833 24.1239) (width 5) (layer "F.Cu") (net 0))
 (segment (start 159.9438 -0.1143) (end 159.9438 61.8998) (width 0.25) (layer "F.Cu") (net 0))
 (segment (start 153.517222 -0.1143) (end 159.9438 -0.1143) (width 0.25) (layer "F.Cu") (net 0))
 (segment (start 139.194586 16.2753) (end 117.5168 16.2753) (width 5) (layer "F.Cu") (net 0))
 (segment (start 95.240742 18.586939) (end 98.21488 15.612801) (width 5) (layer "F.Cu") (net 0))
 (segment (start 146.97835 3.5565) (end 158.967196 15.545346) (width 0.7) (layer "F.Cu") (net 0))
 (segment (start 151.2434 17.367902) (end 151.2434 21.1529) (width 0.7) (layer "F.Cu") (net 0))
 (segment (start 147.950768 38.017396) (end 149.845127 36.123037) (width 0.7) (layer "F.Cu") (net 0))
 (segment (start 159.9438 61.8998) (end 0.0254 61.8998) (width 0.25) (layer "F.Cu") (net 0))
 (segment (start 156.7434 15.867244) (end 156.7434 21.1529) (width 0.7) (layer "F.Cu") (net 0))
 (segment (start 158.967196 23.129104) (end 156.7434 25.3529) (width 0.7) (layer "F.Cu") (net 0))
 (segment (start 139.405803 16.2753) (end 140.604162 15.076941) (width 0.75) (layer "F.Cu") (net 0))
 (segment (start 148.316926 7.44077) (end 156.7434 15.867244) (width 0.7) (layer "F.Cu") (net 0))
 (segment (start 159.9438 -0.1143) (end 160.0708 -0.1143) (width 0.25) (layer "F.Cu") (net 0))
 (segment (start 0.0254 61.8998) (end 0.0254 -0.3048) (width 0.25) (layer "F.Cu") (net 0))
 (segment (start 113.789182 15.612801) (end 117.5168 19.340419) (width 5) (layer "F.Cu") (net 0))
 (segment (start 148.80701 22.91651) (end 151.2434 25.3529) (width 0.7) (layer "F.Cu") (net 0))
 (segment (start 69.717902 -0.1143) (end 153.517222 -0.1143) (width 0.25) (layer "F.Cu") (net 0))
 (segment (start 148.152724 53.943537) (end 63.091466 53.943537) (width 0.75) (layer "F.Cu") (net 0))
 (segment (start 141.301 3.699) (end 146.919297 3.699) (width 0.75) (layer "F.Cu") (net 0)))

